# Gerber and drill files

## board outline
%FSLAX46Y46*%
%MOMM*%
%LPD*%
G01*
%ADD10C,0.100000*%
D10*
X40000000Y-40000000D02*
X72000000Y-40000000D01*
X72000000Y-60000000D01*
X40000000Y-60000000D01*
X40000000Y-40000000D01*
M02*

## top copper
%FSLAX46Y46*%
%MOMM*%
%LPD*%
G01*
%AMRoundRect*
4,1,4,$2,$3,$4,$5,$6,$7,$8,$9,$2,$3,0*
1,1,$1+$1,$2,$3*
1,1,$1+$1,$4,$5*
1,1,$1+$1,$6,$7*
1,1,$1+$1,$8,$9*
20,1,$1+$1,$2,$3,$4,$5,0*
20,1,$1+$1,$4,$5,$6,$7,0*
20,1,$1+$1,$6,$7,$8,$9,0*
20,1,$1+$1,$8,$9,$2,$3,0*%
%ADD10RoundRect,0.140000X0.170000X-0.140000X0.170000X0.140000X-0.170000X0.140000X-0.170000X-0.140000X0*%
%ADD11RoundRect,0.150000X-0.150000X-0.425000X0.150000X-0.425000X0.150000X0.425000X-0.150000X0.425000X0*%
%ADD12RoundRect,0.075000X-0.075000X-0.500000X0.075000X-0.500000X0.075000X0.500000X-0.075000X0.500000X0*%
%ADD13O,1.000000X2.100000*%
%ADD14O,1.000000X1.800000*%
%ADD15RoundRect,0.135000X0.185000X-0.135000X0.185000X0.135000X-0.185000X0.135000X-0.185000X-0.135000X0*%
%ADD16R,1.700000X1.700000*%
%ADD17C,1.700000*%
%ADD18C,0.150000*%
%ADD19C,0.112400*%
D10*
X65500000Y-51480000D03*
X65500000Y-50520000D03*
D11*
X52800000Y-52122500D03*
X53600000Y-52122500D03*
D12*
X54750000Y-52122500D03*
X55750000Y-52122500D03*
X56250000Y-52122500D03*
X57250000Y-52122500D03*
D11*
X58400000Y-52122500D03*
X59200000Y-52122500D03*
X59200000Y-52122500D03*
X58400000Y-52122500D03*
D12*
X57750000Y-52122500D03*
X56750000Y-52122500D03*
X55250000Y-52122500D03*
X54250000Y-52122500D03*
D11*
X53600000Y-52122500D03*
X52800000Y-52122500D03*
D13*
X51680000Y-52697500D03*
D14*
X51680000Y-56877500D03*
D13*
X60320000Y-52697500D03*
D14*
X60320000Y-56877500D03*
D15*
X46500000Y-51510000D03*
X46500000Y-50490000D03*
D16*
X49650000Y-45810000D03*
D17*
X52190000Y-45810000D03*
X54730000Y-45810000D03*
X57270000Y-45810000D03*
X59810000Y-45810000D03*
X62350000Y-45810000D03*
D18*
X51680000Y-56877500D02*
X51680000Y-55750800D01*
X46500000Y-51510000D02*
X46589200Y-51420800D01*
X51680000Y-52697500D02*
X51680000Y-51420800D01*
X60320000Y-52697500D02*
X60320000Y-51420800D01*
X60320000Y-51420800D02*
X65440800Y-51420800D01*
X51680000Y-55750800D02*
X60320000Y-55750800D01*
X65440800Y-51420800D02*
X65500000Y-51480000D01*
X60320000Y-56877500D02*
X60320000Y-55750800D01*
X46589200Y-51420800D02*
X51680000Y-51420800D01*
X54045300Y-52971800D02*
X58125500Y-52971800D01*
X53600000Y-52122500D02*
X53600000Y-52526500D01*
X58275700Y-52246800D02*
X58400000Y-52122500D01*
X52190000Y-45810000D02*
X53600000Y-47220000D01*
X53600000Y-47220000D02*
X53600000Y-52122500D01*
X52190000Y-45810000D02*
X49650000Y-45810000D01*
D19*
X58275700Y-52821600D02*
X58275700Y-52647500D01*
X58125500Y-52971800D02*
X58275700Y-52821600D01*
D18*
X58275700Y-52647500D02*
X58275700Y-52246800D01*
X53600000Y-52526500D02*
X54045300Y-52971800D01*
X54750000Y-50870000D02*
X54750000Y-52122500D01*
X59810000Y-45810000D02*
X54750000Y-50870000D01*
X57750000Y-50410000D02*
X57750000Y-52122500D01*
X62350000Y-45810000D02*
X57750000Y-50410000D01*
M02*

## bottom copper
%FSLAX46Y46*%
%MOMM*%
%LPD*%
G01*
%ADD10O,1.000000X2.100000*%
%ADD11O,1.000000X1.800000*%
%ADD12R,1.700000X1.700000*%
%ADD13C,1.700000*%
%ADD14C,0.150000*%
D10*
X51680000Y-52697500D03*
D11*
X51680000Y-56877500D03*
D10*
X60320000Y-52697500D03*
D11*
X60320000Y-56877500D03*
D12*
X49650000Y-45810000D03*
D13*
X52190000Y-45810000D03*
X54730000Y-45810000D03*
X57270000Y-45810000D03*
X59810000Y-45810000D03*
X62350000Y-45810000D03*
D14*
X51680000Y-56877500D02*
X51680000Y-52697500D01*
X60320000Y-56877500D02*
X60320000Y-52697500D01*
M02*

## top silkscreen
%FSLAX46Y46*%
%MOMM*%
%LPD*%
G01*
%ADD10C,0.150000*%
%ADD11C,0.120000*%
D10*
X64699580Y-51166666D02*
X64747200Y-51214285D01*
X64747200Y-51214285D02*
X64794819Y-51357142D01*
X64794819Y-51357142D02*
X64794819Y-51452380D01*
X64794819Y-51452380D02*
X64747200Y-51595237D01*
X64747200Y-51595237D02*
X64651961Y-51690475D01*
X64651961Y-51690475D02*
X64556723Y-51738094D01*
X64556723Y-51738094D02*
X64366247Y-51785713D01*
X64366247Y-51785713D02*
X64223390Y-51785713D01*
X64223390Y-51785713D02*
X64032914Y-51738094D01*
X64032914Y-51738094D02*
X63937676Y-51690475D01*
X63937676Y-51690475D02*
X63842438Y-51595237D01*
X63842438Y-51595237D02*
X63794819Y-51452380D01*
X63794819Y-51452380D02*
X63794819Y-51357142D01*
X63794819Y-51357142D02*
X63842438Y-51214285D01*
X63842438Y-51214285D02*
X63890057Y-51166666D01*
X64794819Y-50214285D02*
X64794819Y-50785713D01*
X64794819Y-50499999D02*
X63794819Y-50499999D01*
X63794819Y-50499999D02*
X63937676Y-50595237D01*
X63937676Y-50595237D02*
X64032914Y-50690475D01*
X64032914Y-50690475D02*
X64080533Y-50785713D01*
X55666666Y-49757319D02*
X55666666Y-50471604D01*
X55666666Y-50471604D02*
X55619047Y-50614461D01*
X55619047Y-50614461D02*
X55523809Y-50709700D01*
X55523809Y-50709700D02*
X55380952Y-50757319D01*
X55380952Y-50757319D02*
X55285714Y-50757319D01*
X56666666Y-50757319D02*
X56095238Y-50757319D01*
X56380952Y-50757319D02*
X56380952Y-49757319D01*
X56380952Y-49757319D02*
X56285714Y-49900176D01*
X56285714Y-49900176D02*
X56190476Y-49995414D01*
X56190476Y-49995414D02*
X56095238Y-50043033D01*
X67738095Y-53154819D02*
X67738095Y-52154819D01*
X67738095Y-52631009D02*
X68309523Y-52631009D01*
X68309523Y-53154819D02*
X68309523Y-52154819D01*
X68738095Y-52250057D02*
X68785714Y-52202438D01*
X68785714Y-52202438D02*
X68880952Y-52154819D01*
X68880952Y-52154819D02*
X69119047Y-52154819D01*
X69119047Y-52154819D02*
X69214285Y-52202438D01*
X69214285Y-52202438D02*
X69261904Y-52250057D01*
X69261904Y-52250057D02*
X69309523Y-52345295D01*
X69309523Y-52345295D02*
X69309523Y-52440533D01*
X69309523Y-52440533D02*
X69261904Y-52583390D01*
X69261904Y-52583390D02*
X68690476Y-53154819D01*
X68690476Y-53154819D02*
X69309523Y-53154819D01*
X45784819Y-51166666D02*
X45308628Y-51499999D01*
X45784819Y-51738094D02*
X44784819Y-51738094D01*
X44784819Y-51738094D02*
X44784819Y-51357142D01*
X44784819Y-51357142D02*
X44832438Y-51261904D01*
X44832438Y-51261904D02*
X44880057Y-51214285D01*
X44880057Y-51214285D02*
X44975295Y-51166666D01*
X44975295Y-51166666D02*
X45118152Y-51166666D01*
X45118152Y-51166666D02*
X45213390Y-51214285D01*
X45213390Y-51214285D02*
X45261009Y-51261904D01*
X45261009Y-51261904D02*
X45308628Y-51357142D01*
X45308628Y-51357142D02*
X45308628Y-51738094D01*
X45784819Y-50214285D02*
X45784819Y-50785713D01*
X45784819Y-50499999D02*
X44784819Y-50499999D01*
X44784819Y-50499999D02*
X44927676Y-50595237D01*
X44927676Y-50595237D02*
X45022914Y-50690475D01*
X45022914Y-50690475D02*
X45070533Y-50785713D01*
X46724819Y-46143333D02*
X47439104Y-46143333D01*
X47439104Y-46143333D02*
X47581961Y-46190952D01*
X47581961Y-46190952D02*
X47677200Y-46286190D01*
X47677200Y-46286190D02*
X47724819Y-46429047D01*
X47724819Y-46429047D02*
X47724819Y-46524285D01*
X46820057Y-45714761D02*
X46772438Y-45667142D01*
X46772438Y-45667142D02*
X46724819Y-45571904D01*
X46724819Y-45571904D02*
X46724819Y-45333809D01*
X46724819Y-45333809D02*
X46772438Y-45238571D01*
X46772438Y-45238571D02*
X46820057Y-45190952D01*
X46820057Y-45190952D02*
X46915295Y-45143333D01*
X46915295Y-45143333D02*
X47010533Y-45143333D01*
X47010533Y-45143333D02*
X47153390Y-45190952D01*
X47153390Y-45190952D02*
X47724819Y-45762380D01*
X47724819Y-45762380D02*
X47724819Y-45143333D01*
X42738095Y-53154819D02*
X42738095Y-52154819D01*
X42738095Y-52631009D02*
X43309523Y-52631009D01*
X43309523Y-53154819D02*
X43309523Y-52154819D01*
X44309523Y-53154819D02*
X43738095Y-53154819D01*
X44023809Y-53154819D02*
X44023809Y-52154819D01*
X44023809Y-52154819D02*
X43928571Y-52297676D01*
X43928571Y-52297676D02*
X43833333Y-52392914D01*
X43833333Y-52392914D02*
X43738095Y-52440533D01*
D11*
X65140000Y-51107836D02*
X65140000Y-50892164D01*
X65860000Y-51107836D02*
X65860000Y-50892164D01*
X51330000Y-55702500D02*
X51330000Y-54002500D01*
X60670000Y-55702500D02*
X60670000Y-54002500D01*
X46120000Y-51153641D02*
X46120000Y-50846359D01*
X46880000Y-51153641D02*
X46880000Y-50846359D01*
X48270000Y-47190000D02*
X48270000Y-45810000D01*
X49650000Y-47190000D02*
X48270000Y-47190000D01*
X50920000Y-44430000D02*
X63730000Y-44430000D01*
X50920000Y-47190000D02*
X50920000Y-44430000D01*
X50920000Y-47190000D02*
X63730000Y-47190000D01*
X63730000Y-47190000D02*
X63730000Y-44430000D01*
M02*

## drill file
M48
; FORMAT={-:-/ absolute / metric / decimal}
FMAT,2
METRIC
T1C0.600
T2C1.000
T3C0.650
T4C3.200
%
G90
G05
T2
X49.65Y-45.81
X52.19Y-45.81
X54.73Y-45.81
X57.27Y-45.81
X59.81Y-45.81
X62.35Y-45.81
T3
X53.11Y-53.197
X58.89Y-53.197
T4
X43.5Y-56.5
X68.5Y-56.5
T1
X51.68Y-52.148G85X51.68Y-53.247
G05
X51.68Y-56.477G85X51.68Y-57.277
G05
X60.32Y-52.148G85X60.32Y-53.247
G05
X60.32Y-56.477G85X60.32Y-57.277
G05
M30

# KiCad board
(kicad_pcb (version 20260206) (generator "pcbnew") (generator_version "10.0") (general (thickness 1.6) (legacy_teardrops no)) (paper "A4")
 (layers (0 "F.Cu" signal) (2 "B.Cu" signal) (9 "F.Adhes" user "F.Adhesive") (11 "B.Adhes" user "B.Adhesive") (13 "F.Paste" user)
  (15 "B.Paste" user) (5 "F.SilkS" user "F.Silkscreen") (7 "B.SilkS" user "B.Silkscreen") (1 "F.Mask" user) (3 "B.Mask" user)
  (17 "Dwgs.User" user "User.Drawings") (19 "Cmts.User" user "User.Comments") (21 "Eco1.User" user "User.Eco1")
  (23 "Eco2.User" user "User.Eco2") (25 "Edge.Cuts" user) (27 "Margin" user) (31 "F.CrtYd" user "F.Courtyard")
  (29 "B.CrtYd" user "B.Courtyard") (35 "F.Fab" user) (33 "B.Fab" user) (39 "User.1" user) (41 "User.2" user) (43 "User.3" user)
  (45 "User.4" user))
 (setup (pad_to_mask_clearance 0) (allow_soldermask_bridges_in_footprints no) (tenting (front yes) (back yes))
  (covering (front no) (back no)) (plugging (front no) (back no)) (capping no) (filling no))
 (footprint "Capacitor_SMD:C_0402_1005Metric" (layer "F.Cu") (at 65.5 51 90)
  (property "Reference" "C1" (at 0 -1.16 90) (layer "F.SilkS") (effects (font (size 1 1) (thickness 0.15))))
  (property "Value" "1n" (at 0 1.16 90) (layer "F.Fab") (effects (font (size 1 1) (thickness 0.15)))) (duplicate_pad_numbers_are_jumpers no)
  (fp_line (start -0.107836 -0.36) (end 0.107836 -0.36) (stroke (width 0.12) (type solid)) (layer "F.SilkS"))
  (fp_line (start -0.107836 0.36) (end 0.107836 0.36) (stroke (width 0.12) (type solid)) (layer "F.SilkS"))
  (pad "1" smd roundrect (at -0.48 0 90) (size 0.56 0.62) (layers "F.Cu" "F.Mask" "F.Paste") (roundrect_rratio 0.25) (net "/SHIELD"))
  (pad "2" smd roundrect (at 0.48 0 90) (size 0.56 0.62) (layers "F.Cu" "F.Mask" "F.Paste") (roundrect_rratio 0.25) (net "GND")))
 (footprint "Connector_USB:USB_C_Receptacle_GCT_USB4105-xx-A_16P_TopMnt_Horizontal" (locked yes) (layer "F.Cu") (at 56 55.8025)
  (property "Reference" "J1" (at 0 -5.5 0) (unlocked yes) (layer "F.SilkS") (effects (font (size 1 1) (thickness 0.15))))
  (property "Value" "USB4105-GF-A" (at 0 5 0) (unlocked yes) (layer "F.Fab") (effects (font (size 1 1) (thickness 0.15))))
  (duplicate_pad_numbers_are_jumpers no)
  (fp_line (start -4.67 -0.1) (end -4.67 -1.8) (stroke (width 0.12) (type solid)) (layer "F.SilkS"))
  (fp_line (start 4.67 -0.1) (end 4.67 -1.8) (stroke (width 0.12) (type solid)) (layer "F.SilkS"))
  (pad "" np_thru_hole circle (at -2.89 -2.605) (size 0.65 0.65) (drill 0.65) (layers "*.Cu" "*.Mask"))
  (pad "" np_thru_hole circle (at 2.89 -2.605) (size 0.65 0.65) (drill 0.65) (layers "*.Cu" "*.Mask"))
  (pad "A1" smd roundrect (at -3.2 -3.68) (size 0.6 1.15) (layers "F.Cu" "F.Mask" "F.Paste") (roundrect_rratio 0.25) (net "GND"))
  (pad "A4" smd roundrect (at -2.4 -3.68) (size 0.6 1.15) (layers "F.Cu" "F.Mask" "F.Paste") (roundrect_rratio 0.25) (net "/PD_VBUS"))
  (pad "A5" smd roundrect (at -1.25 -3.68) (size 0.3 1.15) (layers "F.Cu" "F.Mask" "F.Paste") (roundrect_rratio 0.25) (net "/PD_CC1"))
  (pad "A6" smd roundrect (at -0.25 -3.68) (size 0.3 1.15) (layers "F.Cu" "F.Mask" "F.Paste") (roundrect_rratio 0.25)
   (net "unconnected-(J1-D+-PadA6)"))
  (pad "A7" smd roundrect (at 0.25 -3.68) (size 0.3 1.15) (layers "F.Cu" "F.Mask" "F.Paste") (roundrect_rratio 0.25)
   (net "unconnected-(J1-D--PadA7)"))
  (pad "A8" smd roundrect (at 1.25 -3.68) (size 0.3 1.15) (layers "F.Cu" "F.Mask" "F.Paste") (roundrect_rratio 0.25)
   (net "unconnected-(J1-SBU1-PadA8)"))
  (pad "A9" smd roundrect (at 2.4 -3.68) (size 0.6 1.15) (layers "F.Cu" "F.Mask" "F.Paste") (roundrect_rratio 0.25) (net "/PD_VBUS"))
  (pad "A12" smd roundrect (at 3.2 -3.68) (size 0.6 1.15) (layers "F.Cu" "F.Mask" "F.Paste") (roundrect_rratio 0.25) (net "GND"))
  (pad "B1" smd roundrect (at 3.2 -3.68) (size 0.6 1.15) (layers "F.Cu" "F.Mask" "F.Paste") (roundrect_rratio 0.25) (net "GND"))
  (pad "B4" smd roundrect (at 2.4 -3.68) (size 0.6 1.15) (layers "F.Cu" "F.Mask" "F.Paste") (roundrect_rratio 0.25) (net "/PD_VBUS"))
  (pad "B5" smd roundrect (at 1.75 -3.68) (size 0.3 1.15) (layers "F.Cu" "F.Mask" "F.Paste") (roundrect_rratio 0.25) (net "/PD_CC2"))
  (pad "B6" smd roundrect (at 0.75 -3.68) (size 0.3 1.15) (layers "F.Cu" "F.Mask" "F.Paste") (roundrect_rratio 0.25)
   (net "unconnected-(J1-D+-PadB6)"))
  (pad "B7" smd roundrect (at -0.75 -3.68) (size 0.3 1.15) (layers "F.Cu" "F.Mask" "F.Paste") (roundrect_rratio 0.25)
   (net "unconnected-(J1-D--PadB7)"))
  (pad "B8" smd roundrect (at -1.75 -3.68) (size 0.3 1.15) (layers "F.Cu" "F.Mask" "F.Paste") (roundrect_rratio 0.25)
   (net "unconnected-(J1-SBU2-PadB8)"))
  (pad "B9" smd roundrect (at -2.4 -3.68) (size 0.6 1.15) (layers "F.Cu" "F.Mask" "F.Paste") (roundrect_rratio 0.25) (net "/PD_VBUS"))
  (pad "B12" smd roundrect (at -3.2 -3.68) (size 0.6 1.15) (layers "F.Cu" "F.Mask" "F.Paste") (roundrect_rratio 0.25) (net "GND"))
  (pad "SH" thru_hole oval (at -4.32 -3.105) (size 1 2.1) (drill oval 0.6 1.7) (layers "*.Cu" "*.Mask" "F.Paste") (remove_unused_layers no)
   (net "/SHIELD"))
  (pad "SH" thru_hole oval (at -4.32 1.075) (size 1 1.8) (drill oval 0.6 1.4) (layers "*.Cu" "*.Mask" "F.Paste") (remove_unused_layers no)
   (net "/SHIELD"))
  (pad "SH" thru_hole oval (at 4.32 -3.105) (size 1 2.1) (drill oval 0.6 1.7) (layers "*.Cu" "*.Mask" "F.Paste") (remove_unused_layers no)
   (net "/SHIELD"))
  (pad "SH" thru_hole oval (at 4.32 1.075) (size 1 1.8) (drill oval 0.6 1.4) (layers "*.Cu" "*.Mask" "F.Paste") (remove_unused_layers no)
   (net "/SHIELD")))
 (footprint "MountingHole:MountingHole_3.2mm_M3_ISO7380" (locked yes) (layer "F.Cu") (at 68.5 56.5)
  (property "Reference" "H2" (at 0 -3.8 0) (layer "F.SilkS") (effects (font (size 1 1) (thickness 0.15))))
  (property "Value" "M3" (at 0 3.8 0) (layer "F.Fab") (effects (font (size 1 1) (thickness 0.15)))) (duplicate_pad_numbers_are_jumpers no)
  (pad "" np_thru_hole circle (at 0 0) (size 3.2 3.2) (drill 3.2) (layers "*.Cu" "*.Mask") (clearance 0.35)))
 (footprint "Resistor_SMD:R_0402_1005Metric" (layer "F.Cu") (at 46.5 51 90)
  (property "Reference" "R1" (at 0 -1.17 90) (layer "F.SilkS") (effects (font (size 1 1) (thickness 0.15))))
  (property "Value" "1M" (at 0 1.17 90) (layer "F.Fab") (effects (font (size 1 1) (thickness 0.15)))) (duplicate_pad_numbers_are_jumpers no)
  (fp_line (start -0.153641 -0.38) (end 0.153641 -0.38) (stroke (width 0.12) (type solid)) (layer "F.SilkS"))
  (fp_line (start -0.153641 0.38) (end 0.153641 0.38) (stroke (width 0.12) (type solid)) (layer "F.SilkS"))
  (pad "1" smd roundrect (at -0.51 0 90) (size 0.54 0.64) (layers "F.Cu" "F.Mask" "F.Paste") (roundrect_rratio 0.25) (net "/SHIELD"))
  (pad "2" smd roundrect (at 0.51 0 90) (size 0.54 0.64) (layers "F.Cu" "F.Mask" "F.Paste") (roundrect_rratio 0.25) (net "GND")))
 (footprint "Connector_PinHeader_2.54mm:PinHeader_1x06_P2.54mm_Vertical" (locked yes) (layer "F.Cu") (at 49.65 45.81 90)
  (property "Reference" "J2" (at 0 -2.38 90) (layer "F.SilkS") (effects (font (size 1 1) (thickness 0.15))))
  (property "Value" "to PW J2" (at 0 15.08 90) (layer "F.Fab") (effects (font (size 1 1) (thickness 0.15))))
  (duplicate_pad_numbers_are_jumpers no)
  (fp_line (start -1.38 -1.38) (end 0 -1.38) (stroke (width 0.12) (type solid)) (layer "F.SilkS"))
  (fp_line (start -1.38 0) (end -1.38 -1.38) (stroke (width 0.12) (type solid)) (layer "F.SilkS"))
  (fp_line (start 1.38 1.27) (end 1.38 14.08) (stroke (width 0.12) (type solid)) (layer "F.SilkS"))
  (fp_line (start -1.38 1.27) (end 1.38 1.27) (stroke (width 0.12) (type solid)) (layer "F.SilkS"))
  (fp_line (start -1.38 1.27) (end -1.38 14.08) (stroke (width 0.12) (type solid)) (layer "F.SilkS"))
  (fp_line (start -1.38 14.08) (end 1.38 14.08) (stroke (width 0.12) (type solid)) (layer "F.SilkS"))
  (pad "1" thru_hole rect (at 0 0 90) (size 1.7 1.7) (drill 1) (layers "*.Cu" "*.Mask") (remove_unused_layers no) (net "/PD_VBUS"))
  (pad "2" thru_hole circle (at 0 2.54 90) (size 1.7 1.7) (drill 1) (layers "*.Cu" "*.Mask") (remove_unused_layers no) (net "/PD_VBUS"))
  (pad "3" thru_hole circle (at 0 5.08 90) (size 1.7 1.7) (drill 1) (layers "*.Cu" "*.Mask") (remove_unused_layers no) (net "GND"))
  (pad "4" thru_hole circle (at 0 7.62 90) (size 1.7 1.7) (drill 1) (layers "*.Cu" "*.Mask") (remove_unused_layers no) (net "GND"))
  (pad "5" thru_hole circle (at 0 10.16 90) (size 1.7 1.7) (drill 1) (layers "*.Cu" "*.Mask") (remove_unused_layers no) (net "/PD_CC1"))
  (pad "6" thru_hole circle (at 0 12.7 90) (size 1.7 1.7) (drill 1) (layers "*.Cu" "*.Mask") (remove_unused_layers no) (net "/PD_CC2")))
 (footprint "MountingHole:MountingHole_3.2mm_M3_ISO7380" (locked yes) (layer "F.Cu") (at 43.5 56.5)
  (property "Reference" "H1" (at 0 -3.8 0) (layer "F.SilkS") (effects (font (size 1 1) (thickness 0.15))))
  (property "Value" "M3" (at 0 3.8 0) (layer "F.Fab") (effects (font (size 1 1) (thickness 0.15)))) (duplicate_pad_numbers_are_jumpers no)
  (pad "" np_thru_hole circle (at 0 0) (size 3.2 3.2) (drill 3.2) (layers "*.Cu" "*.Mask") (clearance 0.35)))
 (gr_rect (start 40 40) (end 72 60) (stroke (width 0.1) (type default)) (fill no) (layer "Edge.Cuts"))
 (segment (start 51.68 56.8775) (end 51.68 55.7508) (width 0.15) (layer "F.Cu") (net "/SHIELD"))
 (segment (start 46.5 51.51) (end 46.5892 51.4208) (width 0.15) (layer "F.Cu") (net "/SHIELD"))
 (segment (start 51.68 52.6975) (end 51.68 51.4208) (width 0.15) (layer "F.Cu") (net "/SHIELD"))
 (segment (start 60.32 52.6975) (end 60.32 51.4208) (width 0.15) (layer "F.Cu") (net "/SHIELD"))
 (segment (start 60.32 51.4208) (end 65.4408 51.4208) (width 0.15) (layer "F.Cu") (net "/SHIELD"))
 (segment (start 51.68 55.7508) (end 60.32 55.7508) (width 0.15) (layer "F.Cu") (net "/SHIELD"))
 (segment (start 65.4408 51.4208) (end 65.5 51.48) (width 0.15) (layer "F.Cu") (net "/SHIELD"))
 (segment (start 60.32 56.8775) (end 60.32 55.7508) (width 0.15) (layer "F.Cu") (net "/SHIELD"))
 (segment (start 46.5892 51.4208) (end 51.68 51.4208) (width 0.15) (layer "F.Cu") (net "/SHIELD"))
 (segment (start 51.68 56.8775) (end 51.68 52.6975) (width 0.15) (layer "B.Cu") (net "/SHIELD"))
 (segment (start 60.32 56.8775) (end 60.32 52.6975) (width 0.15) (layer "B.Cu") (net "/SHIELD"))
 (segment (start 54.0453 52.9718) (end 58.1255 52.9718) (width 0.15) (layer "F.Cu") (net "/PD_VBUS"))
 (segment (start 53.6 52.1225) (end 53.6 52.5265) (width 0.15) (layer "F.Cu") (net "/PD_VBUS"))
 (segment (start 58.2757 52.2468) (end 58.4 52.1225) (width 0.15) (layer "F.Cu") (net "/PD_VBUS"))
 (segment (start 52.19 45.81) (end 53.6 47.22) (width 0.15) (layer "F.Cu") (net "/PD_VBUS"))
 (segment (start 53.6 47.22) (end 53.6 52.1225) (width 0.15) (layer "F.Cu") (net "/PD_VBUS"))
 (segment (start 52.19 45.81) (end 49.65 45.81) (width 0.15) (layer "F.Cu") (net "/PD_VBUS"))
 (segment (start 58.2757 52.8216) (end 58.2757 52.6475) (width 0.1124) (layer "F.Cu") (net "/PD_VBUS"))
 (segment (start 58.1255 52.9718) (end 58.2757 52.8216) (width 0.1124) (layer "F.Cu") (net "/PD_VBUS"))
 (segment (start 58.2757 52.6475) (end 58.2757 52.2468) (width 0.15) (layer "F.Cu") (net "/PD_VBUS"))
 (segment (start 53.6 52.5265) (end 54.0453 52.9718) (width 0.15) (layer "F.Cu") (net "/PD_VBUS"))
 (segment (start 54.75 50.87) (end 54.75 52.1225) (width 0.15) (layer "F.Cu") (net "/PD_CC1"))
 (segment (start 59.81 45.81) (end 54.75 50.87) (width 0.15) (layer "F.Cu") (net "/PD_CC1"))
 (segment (start 57.75 50.41) (end 57.75 52.1225) (width 0.15) (layer "F.Cu") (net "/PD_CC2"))
 (segment (start 62.35 45.81) (end 57.75 50.41) (width 0.15) (layer "F.Cu") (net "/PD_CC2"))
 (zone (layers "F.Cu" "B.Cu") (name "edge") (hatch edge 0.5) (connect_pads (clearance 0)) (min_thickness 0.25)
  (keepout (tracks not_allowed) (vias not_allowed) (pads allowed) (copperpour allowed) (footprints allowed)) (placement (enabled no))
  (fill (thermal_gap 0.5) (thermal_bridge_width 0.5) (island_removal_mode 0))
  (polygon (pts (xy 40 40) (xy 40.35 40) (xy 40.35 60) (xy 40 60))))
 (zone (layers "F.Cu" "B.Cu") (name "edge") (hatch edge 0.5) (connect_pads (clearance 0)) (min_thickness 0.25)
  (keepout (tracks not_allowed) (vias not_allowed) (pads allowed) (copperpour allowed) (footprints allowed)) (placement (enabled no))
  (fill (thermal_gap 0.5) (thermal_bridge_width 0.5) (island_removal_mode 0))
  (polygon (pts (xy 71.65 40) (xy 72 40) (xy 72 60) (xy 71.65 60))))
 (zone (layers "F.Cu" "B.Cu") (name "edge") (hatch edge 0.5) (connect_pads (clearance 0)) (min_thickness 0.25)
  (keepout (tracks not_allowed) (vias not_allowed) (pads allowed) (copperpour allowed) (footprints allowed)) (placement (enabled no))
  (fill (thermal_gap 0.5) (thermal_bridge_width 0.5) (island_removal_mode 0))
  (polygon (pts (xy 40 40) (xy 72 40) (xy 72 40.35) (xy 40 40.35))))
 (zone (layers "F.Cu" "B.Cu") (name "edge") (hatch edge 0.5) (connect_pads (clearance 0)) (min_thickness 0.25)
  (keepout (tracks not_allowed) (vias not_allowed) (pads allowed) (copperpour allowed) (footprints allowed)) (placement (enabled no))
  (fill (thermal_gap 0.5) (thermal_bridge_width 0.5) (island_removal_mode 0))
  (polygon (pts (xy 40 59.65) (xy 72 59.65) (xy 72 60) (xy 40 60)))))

